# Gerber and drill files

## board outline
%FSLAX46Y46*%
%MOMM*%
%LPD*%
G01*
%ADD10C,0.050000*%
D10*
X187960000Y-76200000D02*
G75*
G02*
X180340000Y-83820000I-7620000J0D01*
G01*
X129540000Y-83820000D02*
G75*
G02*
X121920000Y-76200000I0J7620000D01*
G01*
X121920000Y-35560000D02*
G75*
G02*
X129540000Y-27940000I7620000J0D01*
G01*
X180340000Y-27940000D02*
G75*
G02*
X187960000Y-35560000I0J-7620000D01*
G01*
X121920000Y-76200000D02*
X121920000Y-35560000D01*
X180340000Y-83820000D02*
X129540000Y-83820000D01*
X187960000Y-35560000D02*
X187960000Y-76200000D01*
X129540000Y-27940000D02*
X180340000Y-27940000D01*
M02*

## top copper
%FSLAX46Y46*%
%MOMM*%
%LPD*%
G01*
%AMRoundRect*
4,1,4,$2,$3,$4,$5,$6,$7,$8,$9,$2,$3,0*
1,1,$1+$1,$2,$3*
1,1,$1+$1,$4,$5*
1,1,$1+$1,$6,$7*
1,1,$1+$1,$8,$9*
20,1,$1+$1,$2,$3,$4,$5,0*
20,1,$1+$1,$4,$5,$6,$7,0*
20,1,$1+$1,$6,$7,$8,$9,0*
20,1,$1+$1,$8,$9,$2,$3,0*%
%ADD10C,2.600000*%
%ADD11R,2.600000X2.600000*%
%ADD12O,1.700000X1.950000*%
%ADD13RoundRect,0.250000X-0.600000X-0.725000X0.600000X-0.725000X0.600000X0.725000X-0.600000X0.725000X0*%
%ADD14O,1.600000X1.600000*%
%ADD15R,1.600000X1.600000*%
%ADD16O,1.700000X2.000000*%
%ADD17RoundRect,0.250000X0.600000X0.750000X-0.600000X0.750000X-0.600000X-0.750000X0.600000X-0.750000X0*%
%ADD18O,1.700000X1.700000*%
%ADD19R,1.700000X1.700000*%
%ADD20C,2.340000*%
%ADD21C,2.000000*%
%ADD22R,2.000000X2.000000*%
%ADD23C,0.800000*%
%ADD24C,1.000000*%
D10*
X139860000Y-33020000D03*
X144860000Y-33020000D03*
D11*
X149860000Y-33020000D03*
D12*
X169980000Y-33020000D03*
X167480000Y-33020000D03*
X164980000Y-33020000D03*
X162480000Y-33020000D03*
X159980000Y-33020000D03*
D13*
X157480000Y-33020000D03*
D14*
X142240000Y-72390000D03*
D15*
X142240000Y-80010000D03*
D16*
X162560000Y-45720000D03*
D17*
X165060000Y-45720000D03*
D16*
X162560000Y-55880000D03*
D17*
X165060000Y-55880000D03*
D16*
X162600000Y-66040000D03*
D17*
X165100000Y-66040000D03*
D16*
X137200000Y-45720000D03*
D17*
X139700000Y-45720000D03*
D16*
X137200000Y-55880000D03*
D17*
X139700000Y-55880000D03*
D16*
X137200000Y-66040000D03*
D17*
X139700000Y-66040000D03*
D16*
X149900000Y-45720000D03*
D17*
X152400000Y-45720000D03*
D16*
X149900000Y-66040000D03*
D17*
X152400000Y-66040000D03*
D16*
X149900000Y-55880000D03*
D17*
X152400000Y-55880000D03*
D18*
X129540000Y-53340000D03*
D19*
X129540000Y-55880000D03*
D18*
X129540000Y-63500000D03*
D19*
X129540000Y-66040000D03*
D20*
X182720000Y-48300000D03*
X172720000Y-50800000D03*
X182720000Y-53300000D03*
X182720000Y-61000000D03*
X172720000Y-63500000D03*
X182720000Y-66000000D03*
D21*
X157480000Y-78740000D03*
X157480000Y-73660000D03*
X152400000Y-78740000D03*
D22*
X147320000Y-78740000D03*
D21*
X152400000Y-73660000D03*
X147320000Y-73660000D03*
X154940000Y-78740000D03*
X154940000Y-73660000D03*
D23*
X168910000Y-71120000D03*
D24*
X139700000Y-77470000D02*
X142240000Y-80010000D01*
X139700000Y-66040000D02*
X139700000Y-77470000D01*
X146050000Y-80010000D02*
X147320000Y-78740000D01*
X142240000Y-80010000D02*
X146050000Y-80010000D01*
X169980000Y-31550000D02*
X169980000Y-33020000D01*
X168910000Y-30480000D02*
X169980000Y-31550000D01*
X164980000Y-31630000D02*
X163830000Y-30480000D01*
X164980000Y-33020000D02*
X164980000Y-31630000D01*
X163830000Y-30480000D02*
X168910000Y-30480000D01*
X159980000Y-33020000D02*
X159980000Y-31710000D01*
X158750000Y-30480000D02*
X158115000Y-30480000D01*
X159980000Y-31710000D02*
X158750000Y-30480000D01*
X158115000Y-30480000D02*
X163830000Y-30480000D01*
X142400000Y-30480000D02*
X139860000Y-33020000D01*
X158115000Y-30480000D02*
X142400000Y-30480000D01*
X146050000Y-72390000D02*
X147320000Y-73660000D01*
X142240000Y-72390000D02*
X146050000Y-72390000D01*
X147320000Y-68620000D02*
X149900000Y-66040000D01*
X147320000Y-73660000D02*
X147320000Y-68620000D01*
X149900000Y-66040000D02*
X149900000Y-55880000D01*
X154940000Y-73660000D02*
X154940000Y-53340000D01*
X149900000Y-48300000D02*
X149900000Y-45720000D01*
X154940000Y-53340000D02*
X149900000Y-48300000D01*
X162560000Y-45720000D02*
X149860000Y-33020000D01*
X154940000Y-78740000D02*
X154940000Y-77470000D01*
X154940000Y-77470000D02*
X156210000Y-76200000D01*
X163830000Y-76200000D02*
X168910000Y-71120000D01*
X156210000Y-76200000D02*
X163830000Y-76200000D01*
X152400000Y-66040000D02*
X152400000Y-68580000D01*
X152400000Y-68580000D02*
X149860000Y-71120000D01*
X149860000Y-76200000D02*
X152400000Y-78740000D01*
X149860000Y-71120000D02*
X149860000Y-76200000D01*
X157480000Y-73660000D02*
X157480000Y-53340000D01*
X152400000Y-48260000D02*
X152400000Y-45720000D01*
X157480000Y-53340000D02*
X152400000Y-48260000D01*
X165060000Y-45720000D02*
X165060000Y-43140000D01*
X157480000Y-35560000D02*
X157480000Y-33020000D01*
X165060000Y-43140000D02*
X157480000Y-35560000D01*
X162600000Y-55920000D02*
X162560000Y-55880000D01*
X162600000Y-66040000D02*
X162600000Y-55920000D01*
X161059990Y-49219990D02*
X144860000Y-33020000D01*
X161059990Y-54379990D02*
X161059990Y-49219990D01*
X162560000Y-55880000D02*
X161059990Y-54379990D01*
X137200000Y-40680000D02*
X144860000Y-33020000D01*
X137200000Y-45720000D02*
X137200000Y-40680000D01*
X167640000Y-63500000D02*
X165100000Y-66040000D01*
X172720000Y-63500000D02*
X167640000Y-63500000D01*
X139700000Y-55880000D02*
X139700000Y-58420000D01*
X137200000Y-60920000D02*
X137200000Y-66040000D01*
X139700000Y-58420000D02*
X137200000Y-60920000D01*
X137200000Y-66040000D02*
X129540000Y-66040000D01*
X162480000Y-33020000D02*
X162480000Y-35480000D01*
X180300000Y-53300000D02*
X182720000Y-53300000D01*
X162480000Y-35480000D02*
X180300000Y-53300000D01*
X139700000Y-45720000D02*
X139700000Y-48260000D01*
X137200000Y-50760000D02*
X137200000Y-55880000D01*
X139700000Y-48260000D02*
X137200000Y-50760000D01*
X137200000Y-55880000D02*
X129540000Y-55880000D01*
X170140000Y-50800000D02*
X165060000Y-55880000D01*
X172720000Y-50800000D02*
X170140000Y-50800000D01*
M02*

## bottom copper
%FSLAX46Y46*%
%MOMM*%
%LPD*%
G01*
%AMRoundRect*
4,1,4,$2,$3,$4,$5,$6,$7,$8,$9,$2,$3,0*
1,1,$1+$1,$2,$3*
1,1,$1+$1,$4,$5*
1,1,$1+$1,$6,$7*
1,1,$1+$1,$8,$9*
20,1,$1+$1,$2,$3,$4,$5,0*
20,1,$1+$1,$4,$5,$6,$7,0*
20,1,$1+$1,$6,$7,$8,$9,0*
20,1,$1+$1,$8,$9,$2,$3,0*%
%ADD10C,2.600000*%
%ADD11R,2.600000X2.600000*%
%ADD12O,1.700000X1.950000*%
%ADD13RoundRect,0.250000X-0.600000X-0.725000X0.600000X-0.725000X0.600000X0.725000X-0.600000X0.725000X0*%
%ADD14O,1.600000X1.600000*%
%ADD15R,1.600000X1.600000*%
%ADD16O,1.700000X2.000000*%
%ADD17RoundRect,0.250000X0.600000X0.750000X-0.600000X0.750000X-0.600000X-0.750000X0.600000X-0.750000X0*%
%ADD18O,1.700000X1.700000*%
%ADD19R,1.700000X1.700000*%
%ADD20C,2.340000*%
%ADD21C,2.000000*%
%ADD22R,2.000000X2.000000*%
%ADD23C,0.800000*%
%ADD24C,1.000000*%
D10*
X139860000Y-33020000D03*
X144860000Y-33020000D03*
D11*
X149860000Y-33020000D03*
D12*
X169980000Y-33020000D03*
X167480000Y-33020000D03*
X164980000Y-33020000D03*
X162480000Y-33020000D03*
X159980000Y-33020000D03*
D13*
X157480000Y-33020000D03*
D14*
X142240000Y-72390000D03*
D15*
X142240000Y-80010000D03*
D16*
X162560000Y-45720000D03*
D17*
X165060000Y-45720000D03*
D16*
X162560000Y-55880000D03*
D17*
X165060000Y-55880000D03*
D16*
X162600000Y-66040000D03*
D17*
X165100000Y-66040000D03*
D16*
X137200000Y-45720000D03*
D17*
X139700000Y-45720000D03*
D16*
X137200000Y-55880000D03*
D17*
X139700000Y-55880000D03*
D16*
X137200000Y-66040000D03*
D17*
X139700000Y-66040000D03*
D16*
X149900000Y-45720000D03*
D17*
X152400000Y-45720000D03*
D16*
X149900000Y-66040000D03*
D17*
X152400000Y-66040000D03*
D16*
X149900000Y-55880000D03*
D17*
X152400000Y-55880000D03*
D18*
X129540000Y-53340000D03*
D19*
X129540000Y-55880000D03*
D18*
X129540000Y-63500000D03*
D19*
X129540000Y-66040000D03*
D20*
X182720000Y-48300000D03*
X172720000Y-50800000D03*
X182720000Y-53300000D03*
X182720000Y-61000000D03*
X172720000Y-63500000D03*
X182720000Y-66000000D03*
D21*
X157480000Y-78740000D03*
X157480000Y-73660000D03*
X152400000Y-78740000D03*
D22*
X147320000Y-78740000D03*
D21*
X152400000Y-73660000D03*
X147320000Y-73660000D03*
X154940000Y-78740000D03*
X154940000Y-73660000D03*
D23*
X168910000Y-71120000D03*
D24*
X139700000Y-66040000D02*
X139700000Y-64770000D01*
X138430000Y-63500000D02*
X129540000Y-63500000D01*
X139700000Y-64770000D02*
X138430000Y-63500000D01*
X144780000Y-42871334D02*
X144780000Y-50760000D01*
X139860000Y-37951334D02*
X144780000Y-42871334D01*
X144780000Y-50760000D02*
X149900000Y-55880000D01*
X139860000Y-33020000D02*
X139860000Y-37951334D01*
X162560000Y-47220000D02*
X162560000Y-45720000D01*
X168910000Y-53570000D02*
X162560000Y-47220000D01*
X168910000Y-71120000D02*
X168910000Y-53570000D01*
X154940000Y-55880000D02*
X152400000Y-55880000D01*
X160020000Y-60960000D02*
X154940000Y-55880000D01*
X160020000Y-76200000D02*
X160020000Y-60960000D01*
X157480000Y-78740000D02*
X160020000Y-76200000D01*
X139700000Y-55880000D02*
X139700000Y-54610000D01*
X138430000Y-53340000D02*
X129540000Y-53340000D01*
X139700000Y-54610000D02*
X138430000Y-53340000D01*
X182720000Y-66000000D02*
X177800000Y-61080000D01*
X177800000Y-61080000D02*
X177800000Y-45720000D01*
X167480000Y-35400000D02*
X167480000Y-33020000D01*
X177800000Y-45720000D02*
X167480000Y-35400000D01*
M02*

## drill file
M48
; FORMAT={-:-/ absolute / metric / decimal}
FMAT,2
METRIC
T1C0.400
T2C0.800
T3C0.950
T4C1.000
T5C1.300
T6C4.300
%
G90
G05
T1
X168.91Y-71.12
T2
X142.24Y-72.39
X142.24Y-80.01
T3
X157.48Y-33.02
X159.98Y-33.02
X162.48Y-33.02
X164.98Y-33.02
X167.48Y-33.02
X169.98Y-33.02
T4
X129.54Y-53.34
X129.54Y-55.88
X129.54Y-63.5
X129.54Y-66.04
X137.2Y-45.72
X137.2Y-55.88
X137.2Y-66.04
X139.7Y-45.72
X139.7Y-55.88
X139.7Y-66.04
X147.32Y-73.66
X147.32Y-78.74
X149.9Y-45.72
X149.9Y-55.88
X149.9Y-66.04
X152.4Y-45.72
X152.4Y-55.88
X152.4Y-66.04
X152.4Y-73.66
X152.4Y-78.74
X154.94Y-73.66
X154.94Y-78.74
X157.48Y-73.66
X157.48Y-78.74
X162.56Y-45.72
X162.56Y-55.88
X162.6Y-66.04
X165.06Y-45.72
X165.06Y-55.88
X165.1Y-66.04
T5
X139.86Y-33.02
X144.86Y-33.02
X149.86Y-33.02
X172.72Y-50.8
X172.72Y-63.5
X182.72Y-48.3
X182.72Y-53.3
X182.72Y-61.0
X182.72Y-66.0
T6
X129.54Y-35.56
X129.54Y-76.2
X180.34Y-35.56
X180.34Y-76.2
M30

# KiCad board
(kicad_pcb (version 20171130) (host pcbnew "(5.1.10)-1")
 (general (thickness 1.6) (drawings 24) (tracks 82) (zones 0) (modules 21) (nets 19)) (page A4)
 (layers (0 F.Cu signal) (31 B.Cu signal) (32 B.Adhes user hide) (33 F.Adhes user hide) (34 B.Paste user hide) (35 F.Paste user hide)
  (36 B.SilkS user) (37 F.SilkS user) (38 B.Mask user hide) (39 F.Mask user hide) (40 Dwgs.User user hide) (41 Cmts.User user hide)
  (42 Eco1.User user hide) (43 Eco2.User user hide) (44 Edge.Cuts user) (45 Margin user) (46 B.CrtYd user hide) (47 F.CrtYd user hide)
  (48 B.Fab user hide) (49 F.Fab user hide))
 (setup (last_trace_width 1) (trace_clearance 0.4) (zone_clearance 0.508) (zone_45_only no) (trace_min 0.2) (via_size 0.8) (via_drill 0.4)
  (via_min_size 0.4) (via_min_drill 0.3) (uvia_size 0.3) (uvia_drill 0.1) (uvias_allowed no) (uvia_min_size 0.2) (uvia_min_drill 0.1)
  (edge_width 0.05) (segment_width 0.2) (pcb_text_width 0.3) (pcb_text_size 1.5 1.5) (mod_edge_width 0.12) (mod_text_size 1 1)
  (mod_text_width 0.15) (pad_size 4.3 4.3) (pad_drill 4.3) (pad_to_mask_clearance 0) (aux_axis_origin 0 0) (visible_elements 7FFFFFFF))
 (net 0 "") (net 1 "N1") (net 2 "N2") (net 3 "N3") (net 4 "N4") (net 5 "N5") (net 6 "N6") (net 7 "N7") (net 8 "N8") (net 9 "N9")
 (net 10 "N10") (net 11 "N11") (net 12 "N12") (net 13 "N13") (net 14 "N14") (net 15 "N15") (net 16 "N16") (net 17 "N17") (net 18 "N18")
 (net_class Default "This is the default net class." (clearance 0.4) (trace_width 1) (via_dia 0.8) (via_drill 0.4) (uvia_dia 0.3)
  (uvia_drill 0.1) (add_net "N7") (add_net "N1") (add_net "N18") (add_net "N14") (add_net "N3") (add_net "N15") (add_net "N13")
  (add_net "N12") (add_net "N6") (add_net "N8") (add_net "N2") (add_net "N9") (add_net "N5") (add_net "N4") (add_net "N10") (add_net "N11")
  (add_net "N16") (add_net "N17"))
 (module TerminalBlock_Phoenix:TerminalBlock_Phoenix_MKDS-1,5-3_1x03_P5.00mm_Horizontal (layer F.Cu) (at 149.86 33.02 180)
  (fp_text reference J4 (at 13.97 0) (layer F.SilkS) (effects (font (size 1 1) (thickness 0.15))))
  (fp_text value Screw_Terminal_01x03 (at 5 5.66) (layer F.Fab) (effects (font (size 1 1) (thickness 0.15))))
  (pad 3 thru_hole circle (at 10 0 180) (size 2.6 2.6) (drill 1.3) (layers *.Cu *.Mask) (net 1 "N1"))
  (pad 2 thru_hole circle (at 5 0 180) (size 2.6 2.6) (drill 1.3) (layers *.Cu *.Mask) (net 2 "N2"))
  (pad 1 thru_hole rect (at 0 0 180) (size 2.6 2.6) (drill 1.3) (layers *.Cu *.Mask) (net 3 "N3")))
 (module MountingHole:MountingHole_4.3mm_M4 (layer F.Cu) (at 180.34 76.2)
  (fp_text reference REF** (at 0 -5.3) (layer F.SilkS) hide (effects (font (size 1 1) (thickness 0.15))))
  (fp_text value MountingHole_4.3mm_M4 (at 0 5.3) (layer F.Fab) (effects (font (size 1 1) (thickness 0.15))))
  (pad 1 np_thru_hole circle (at 0 0) (size 4.3 4.3) (drill 4.3) (layers *.Cu *.Mask)))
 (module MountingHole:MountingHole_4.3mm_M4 (layer F.Cu) (at 129.54 76.2)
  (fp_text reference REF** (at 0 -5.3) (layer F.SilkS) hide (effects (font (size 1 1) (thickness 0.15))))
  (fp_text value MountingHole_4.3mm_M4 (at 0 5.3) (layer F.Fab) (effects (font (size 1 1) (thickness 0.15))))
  (pad 1 np_thru_hole circle (at 0 0) (size 4.3 4.3) (drill 4.3) (layers *.Cu *.Mask)))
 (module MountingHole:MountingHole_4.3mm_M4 (layer F.Cu) (at 129.54 35.56)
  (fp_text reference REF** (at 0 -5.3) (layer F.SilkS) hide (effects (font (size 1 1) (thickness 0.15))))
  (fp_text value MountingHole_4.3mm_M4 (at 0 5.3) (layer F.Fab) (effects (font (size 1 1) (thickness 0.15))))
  (pad 1 np_thru_hole circle (at 0 0) (size 4.3 4.3) (drill 4.3) (layers *.Cu *.Mask)))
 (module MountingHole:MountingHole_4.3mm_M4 (layer F.Cu) (at 180.34 35.56)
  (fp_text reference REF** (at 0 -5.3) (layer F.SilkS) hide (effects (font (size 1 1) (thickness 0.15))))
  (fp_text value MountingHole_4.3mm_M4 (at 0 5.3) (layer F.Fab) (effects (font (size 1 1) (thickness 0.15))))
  (pad 1 np_thru_hole circle (at 0 0) (size 4.3 4.3) (drill 4.3) (layers *.Cu *.Mask)))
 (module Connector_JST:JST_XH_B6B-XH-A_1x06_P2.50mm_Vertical (layer F.Cu) (at 157.48 33.02)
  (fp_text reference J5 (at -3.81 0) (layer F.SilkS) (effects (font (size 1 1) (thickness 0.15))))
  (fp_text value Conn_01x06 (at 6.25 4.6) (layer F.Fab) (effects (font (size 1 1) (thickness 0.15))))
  (pad 6 thru_hole oval (at 12.5 0) (size 1.7 1.95) (drill 0.95) (layers *.Cu *.Mask) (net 1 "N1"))
  (pad 5 thru_hole oval (at 10 0) (size 1.7 1.95) (drill 0.95) (layers *.Cu *.Mask) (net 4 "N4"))
  (pad 4 thru_hole oval (at 7.5 0) (size 1.7 1.95) (drill 0.95) (layers *.Cu *.Mask) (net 1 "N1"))
  (pad 3 thru_hole oval (at 5 0) (size 1.7 1.95) (drill 0.95) (layers *.Cu *.Mask) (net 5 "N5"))
  (pad 2 thru_hole oval (at 2.5 0) (size 1.7 1.95) (drill 0.95) (layers *.Cu *.Mask) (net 1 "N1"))
  (pad 1 thru_hole roundrect (at 0 0) (size 1.7 1.95) (drill 0.95) (layers *.Cu *.Mask) (roundrect_rratio 0.147059) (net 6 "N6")))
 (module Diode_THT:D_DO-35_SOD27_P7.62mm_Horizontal (layer F.Cu) (at 142.24 80.01 90)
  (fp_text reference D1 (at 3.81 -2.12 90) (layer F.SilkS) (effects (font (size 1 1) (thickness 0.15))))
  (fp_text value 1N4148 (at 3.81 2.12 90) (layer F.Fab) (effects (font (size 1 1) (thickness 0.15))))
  (pad 2 thru_hole oval (at 7.62 0 90) (size 1.6 1.6) (drill 0.8) (layers *.Cu *.Mask) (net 1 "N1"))
  (pad 1 thru_hole rect (at 0 0 90) (size 1.6 1.6) (drill 0.8) (layers *.Cu *.Mask) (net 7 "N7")))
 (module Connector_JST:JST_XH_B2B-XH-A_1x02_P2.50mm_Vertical (layer F.Cu) (at 165.06 45.72 180)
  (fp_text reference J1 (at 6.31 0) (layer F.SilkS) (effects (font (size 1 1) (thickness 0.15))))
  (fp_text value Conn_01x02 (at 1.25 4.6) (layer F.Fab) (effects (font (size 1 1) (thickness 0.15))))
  (pad 2 thru_hole oval (at 2.5 0 180) (size 1.7 2) (drill 1) (layers *.Cu *.Mask) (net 3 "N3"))
  (pad 1 thru_hole roundrect (at 0 0 180) (size 1.7 2) (drill 1) (layers *.Cu *.Mask) (roundrect_rratio 0.147059) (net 6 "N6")))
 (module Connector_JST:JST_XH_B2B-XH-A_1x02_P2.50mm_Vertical (layer F.Cu) (at 165.06 55.88 180)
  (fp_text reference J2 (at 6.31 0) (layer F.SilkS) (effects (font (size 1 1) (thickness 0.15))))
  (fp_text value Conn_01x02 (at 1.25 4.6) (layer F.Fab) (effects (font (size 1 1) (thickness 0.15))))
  (pad 2 thru_hole oval (at 2.5 0 180) (size 1.7 2) (drill 1) (layers *.Cu *.Mask) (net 2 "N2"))
  (pad 1 thru_hole roundrect (at 0 0 180) (size 1.7 2) (drill 1) (layers *.Cu *.Mask) (roundrect_rratio 0.147059) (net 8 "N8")))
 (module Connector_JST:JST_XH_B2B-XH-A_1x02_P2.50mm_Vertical (layer F.Cu) (at 165.1 66.04 180)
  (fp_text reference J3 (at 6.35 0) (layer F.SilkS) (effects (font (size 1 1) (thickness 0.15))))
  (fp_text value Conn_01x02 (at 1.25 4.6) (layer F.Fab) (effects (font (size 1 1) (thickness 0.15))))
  (pad 2 thru_hole oval (at 2.5 0 180) (size 1.7 2) (drill 1) (layers *.Cu *.Mask) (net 2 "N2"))
  (pad 1 thru_hole roundrect (at 0 0 180) (size 1.7 2) (drill 1) (layers *.Cu *.Mask) (roundrect_rratio 0.147059) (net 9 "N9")))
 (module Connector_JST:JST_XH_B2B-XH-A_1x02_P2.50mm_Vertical (layer F.Cu) (at 139.7 45.72 180)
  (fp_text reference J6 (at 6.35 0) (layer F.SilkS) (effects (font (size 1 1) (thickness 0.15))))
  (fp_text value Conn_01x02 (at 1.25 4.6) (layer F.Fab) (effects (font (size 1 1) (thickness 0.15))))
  (pad 2 thru_hole oval (at 2.5 0 180) (size 1.7 2) (drill 1) (layers *.Cu *.Mask) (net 2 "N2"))
  (pad 1 thru_hole roundrect (at 0 0 180) (size 1.7 2) (drill 1) (layers *.Cu *.Mask) (roundrect_rratio 0.147059) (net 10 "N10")))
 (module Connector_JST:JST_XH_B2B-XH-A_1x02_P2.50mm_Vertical (layer F.Cu) (at 139.7 55.88 180)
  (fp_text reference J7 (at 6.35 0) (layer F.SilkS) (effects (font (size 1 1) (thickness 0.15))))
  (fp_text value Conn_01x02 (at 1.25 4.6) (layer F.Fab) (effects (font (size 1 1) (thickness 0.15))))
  (pad 2 thru_hole oval (at 2.5 0 180) (size 1.7 2) (drill 1) (layers *.Cu *.Mask) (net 10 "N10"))
  (pad 1 thru_hole roundrect (at 0 0 180) (size 1.7 2) (drill 1) (layers *.Cu *.Mask) (roundrect_rratio 0.147059) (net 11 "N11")))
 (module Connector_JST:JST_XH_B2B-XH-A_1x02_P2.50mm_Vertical (layer F.Cu) (at 139.7 66.04 180)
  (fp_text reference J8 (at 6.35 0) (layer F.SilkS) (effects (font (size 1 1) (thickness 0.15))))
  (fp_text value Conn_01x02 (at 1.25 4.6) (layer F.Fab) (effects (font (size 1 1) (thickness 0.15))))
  (pad 2 thru_hole oval (at 2.5 0 180) (size 1.7 2) (drill 1) (layers *.Cu *.Mask) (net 11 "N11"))
  (pad 1 thru_hole roundrect (at 0 0 180) (size 1.7 2) (drill 1) (layers *.Cu *.Mask) (roundrect_rratio 0.147059) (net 7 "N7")))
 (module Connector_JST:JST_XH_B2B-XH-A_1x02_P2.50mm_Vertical (layer F.Cu) (at 152.4 45.72 180)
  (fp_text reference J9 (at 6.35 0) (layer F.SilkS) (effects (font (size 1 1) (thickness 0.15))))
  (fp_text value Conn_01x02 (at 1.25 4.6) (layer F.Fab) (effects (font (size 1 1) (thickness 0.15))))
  (pad 2 thru_hole oval (at 2.5 0 180) (size 1.7 2) (drill 1) (layers *.Cu *.Mask) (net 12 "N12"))
  (pad 1 thru_hole roundrect (at 0 0 180) (size 1.7 2) (drill 1) (layers *.Cu *.Mask) (roundrect_rratio 0.147059) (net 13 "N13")))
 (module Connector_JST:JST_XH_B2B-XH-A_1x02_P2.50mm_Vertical (layer F.Cu) (at 152.4 66.04 180)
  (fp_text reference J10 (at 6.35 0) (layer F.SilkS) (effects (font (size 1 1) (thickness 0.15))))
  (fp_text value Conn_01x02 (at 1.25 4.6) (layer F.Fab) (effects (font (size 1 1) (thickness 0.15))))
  (pad 2 thru_hole oval (at 2.5 0 180) (size 1.7 2) (drill 1) (layers *.Cu *.Mask) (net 1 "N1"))
  (pad 1 thru_hole roundrect (at 0 0 180) (size 1.7 2) (drill 1) (layers *.Cu *.Mask) (roundrect_rratio 0.147059) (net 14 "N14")))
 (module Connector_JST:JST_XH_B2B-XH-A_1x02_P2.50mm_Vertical (layer F.Cu) (at 152.4 55.88 180)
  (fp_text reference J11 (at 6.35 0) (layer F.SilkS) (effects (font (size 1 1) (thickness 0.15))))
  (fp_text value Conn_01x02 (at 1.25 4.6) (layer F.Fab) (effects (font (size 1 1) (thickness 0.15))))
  (pad 2 thru_hole oval (at 2.5 0 180) (size 1.7 2) (drill 1) (layers *.Cu *.Mask) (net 1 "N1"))
  (pad 1 thru_hole roundrect (at 0 0 180) (size 1.7 2) (drill 1) (layers *.Cu *.Mask) (roundrect_rratio 0.147059) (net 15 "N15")))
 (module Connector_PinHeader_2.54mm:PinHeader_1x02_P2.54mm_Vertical (layer F.Cu) (at 129.54 55.88 180)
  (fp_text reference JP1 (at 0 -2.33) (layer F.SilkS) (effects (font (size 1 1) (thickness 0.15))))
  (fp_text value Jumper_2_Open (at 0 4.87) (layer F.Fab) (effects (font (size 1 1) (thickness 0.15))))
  (pad 2 thru_hole oval (at 0 2.54 180) (size 1.7 1.7) (drill 1) (layers *.Cu *.Mask) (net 11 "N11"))
  (pad 1 thru_hole rect (at 0 0 180) (size 1.7 1.7) (drill 1) (layers *.Cu *.Mask) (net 10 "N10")))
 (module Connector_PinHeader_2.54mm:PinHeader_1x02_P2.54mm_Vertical (layer F.Cu) (at 129.54 66.04 180)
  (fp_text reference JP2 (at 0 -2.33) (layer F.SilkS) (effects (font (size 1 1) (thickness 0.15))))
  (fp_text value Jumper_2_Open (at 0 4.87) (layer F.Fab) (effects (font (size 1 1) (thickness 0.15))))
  (pad 2 thru_hole oval (at 0 2.54 180) (size 1.7 1.7) (drill 1) (layers *.Cu *.Mask) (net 7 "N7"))
  (pad 1 thru_hole rect (at 0 0 180) (size 1.7 1.7) (drill 1) (layers *.Cu *.Mask) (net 11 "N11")))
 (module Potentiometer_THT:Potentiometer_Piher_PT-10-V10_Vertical (layer F.Cu) (at 182.72 48.3 180)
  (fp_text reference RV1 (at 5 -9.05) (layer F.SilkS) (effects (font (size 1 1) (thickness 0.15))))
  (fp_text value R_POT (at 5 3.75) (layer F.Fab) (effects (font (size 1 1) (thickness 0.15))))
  (pad 1 thru_hole circle (at 0 0 180) (size 2.34 2.34) (drill 1.3) (layers *.Cu *.Mask) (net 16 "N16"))
  (pad 2 thru_hole circle (at 10 -2.5 180) (size 2.34 2.34) (drill 1.3) (layers *.Cu *.Mask) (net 8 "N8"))
  (pad 3 thru_hole circle (at 0 -5 180) (size 2.34 2.34) (drill 1.3) (layers *.Cu *.Mask) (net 5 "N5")))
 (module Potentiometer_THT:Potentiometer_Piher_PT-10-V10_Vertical (layer F.Cu) (at 182.72 61 180)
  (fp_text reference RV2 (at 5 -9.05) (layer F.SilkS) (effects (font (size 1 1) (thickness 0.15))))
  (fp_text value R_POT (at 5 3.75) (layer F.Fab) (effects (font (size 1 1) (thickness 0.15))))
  (pad 1 thru_hole circle (at 0 0 180) (size 2.34 2.34) (drill 1.3) (layers *.Cu *.Mask) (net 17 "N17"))
  (pad 2 thru_hole circle (at 10 -2.5 180) (size 2.34 2.34) (drill 1.3) (layers *.Cu *.Mask) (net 9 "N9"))
  (pad 3 thru_hole circle (at 0 -5 180) (size 2.34 2.34) (drill 1.3) (layers *.Cu *.Mask) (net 4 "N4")))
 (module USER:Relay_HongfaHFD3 (layer F.Cu) (at 147.32 78.74 90)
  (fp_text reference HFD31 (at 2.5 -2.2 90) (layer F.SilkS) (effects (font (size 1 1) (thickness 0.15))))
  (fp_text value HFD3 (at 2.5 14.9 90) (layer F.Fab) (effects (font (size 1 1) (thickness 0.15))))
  (pad 5 thru_hole circle (at 0 10.16 90) (size 2 2) (drill 1) (layers *.Cu *.Mask) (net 15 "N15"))
  (pad 8 thru_hole circle (at 5.08 10.16 90) (size 2 2) (drill 1) (layers *.Cu *.Mask) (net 13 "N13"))
  (pad 3 thru_hole circle (at 0 5.08 90) (size 2 2) (drill 1) (layers *.Cu *.Mask) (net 14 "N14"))
  (pad 1 thru_hole rect (at 0 0 90) (size 2 2) (drill 1) (layers *.Cu *.Mask) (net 7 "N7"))
  (pad 10 thru_hole circle (at 5.08 5.08 90) (size 2 2) (drill 1) (layers *.Cu *.Mask) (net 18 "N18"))
  (pad 12 thru_hole circle (at 5.08 0 90) (size 2 2) (drill 1) (layers *.Cu *.Mask) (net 1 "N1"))
  (pad 4 thru_hole circle (at 0 7.62) (size 2 2) (drill 1) (layers *.Cu *.Mask) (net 3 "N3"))
  (pad 9 thru_hole circle (at 5.08 7.62) (size 2 2) (drill 1) (layers *.Cu *.Mask) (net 12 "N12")))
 (gr_arc (start 180.34 76.2) (end 180.34 83.82) (angle -90) (layer Edge.Cuts) (width 0.05))
 (gr_arc (start 129.54 76.2) (end 121.92 76.2) (angle -90) (layer Edge.Cuts) (width 0.05))
 (gr_arc (start 129.54 35.56) (end 129.54 27.94) (angle -90) (layer Edge.Cuts) (width 0.05))
 (gr_arc (start 180.34 35.56) (end 187.96 35.56) (angle -90) (layer Edge.Cuts) (width 0.05))
 (gr_line (start 121.92 76.2) (end 121.92 35.56) (layer Edge.Cuts) (width 0.05))
 (gr_line (start 180.34 83.82) (end 129.54 83.82) (layer Edge.Cuts) (width 0.05))
 (gr_line (start 187.96 35.56) (end 187.96 76.2) (layer Edge.Cuts) (width 0.05))
 (gr_line (start 129.54 27.94) (end 180.34 27.94) (layer Edge.Cuts) (width 0.05))
 (segment (start 139.7 77.47) (end 142.24 80.01) (width 1) (layer F.Cu) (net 7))
 (segment (start 139.7 66.04) (end 139.7 77.47) (width 1) (layer F.Cu) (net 7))
 (segment (start 146.05 80.01) (end 147.32 78.74) (width 1) (layer F.Cu) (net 7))
 (segment (start 142.24 80.01) (end 146.05 80.01) (width 1) (layer F.Cu) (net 7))
 (segment (start 139.7 66.04) (end 139.7 64.77) (width 1) (layer B.Cu) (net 7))
 (segment (start 138.43 63.5) (end 129.54 63.5) (width 1) (layer B.Cu) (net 7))
 (segment (start 139.7 64.77) (end 138.43 63.5) (width 1) (layer B.Cu) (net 7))
 (segment (start 169.98 31.55) (end 169.98 33.02) (width 1) (layer F.Cu) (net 1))
 (segment (start 168.91 30.48) (end 169.98 31.55) (width 1) (layer F.Cu) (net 1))
 (segment (start 164.98 31.63) (end 163.83 30.48) (width 1) (layer F.Cu) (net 1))
 (segment (start 164.98 33.02) (end 164.98 31.63) (width 1) (layer F.Cu) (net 1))
 (segment (start 163.83 30.48) (end 168.91 30.48) (width 1) (layer F.Cu) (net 1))
 (segment (start 159.98 33.02) (end 159.98 31.71) (width 1) (layer F.Cu) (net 1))
 (segment (start 158.75 30.48) (end 158.115 30.48) (width 1) (layer F.Cu) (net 1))
 (segment (start 159.98 31.71) (end 158.75 30.48) (width 1) (layer F.Cu) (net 1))
 (segment (start 158.115 30.48) (end 163.83 30.48) (width 1) (layer F.Cu) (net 1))
 (segment (start 142.4 30.48) (end 139.86 33.02) (width 1) (layer F.Cu) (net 1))
 (segment (start 158.115 30.48) (end 142.4 30.48) (width 1) (layer F.Cu) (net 1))
 (segment (start 146.05 72.39) (end 147.32 73.66) (width 1) (layer F.Cu) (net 1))
 (segment (start 142.24 72.39) (end 146.05 72.39) (width 1) (layer F.Cu) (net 1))
 (segment (start 147.32 68.62) (end 149.9 66.04) (width 1) (layer F.Cu) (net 1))
 (segment (start 147.32 73.66) (end 147.32 68.62) (width 1) (layer F.Cu) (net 1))
 (segment (start 149.9 66.04) (end 149.9 55.88) (width 1) (layer F.Cu) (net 1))
 (segment (start 144.78 42.871334) (end 144.78 50.76) (width 1) (layer B.Cu) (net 1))
 (segment (start 139.86 37.951334) (end 144.78 42.871334) (width 1) (layer B.Cu) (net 1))
 (segment (start 144.78 50.76) (end 149.9 55.88) (width 1) (layer B.Cu) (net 1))
 (segment (start 139.86 33.02) (end 139.86 37.951334) (width 1) (layer B.Cu) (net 1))
 (segment (start 154.94 73.66) (end 154.94 53.34) (width 1) (layer F.Cu) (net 12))
 (segment (start 149.9 48.3) (end 149.9 45.72) (width 1) (layer F.Cu) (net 12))
 (segment (start 154.94 53.34) (end 149.9 48.3) (width 1) (layer F.Cu) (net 12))
 (segment (start 162.56 45.72) (end 149.86 33.02) (width 1) (layer F.Cu) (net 3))
 (segment (start 154.94 78.74) (end 154.94 77.47) (width 1) (layer F.Cu) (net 3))
 (segment (start 154.94 77.47) (end 156.21 76.2) (width 1) (layer F.Cu) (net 3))
 (via (at 168.91 71.12) (size 0.8) (drill 0.4) (layers F.Cu B.Cu) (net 3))
 (segment (start 163.83 76.2) (end 168.91 71.12) (width 1) (layer F.Cu) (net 3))
 (segment (start 156.21 76.2) (end 163.83 76.2) (width 1) (layer F.Cu) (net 3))
 (segment (start 162.56 47.22) (end 162.56 45.72) (width 1) (layer B.Cu) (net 3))
 (segment (start 168.91 53.57) (end 162.56 47.22) (width 1) (layer B.Cu) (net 3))
 (segment (start 168.91 71.12) (end 168.91 53.57) (width 1) (layer B.Cu) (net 3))
 (segment (start 152.4 66.04) (end 152.4 68.58) (width 1) (layer F.Cu) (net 14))
 (segment (start 152.4 68.58) (end 149.86 71.12) (width 1) (layer F.Cu) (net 14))
 (segment (start 149.86 76.2) (end 152.4 78.74) (width 1) (layer F.Cu) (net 14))
 (segment (start 149.86 71.12) (end 149.86 76.2) (width 1) (layer F.Cu) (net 14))
 (segment (start 157.48 73.66) (end 157.48 53.34) (width 1) (layer F.Cu) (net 13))
 (segment (start 152.4 48.26) (end 152.4 45.72) (width 1) (layer F.Cu) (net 13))
 (segment (start 157.48 53.34) (end 152.4 48.26) (width 1) (layer F.Cu) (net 13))
 (segment (start 154.94 55.88) (end 152.4 55.88) (width 1) (layer B.Cu) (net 15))
 (segment (start 160.02 60.96) (end 154.94 55.88) (width 1) (layer B.Cu) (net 15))
 (segment (start 160.02 76.2) (end 160.02 60.96) (width 1) (layer B.Cu) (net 15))
 (segment (start 157.48 78.74) (end 160.02 76.2) (width 1) (layer B.Cu) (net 15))
 (segment (start 165.06 45.72) (end 165.06 43.14) (width 1) (layer F.Cu) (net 6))
 (segment (start 157.48 35.56) (end 157.48 33.02) (width 1) (layer F.Cu) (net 6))
 (segment (start 165.06 43.14) (end 157.48 35.56) (width 1) (layer F.Cu) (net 6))
 (segment (start 162.6 55.92) (end 162.56 55.88) (width 1) (layer F.Cu) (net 2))
 (segment (start 162.6 66.04) (end 162.6 55.92) (width 1) (layer F.Cu) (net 2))
 (segment (start 161.05999 49.21999) (end 144.86 33.02) (width 1) (layer F.Cu) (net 2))
 (segment (start 161.05999 54.37999) (end 161.05999 49.21999) (width 1) (layer F.Cu) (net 2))
 (segment (start 162.56 55.88) (end 161.05999 54.37999) (width 1) (layer F.Cu) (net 2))
 (segment (start 137.2 40.68) (end 144.86 33.02) (width 1) (layer F.Cu) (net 2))
 (segment (start 137.2 45.72) (end 137.2 40.68) (width 1) (layer F.Cu) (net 2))
 (segment (start 167.64 63.5) (end 165.1 66.04) (width 1) (layer F.Cu) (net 9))
 (segment (start 172.72 63.5) (end 167.64 63.5) (width 1) (layer F.Cu) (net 9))
 (segment (start 139.7 55.88) (end 139.7 58.42) (width 1) (layer F.Cu) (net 11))
 (segment (start 137.2 60.92) (end 137.2 66.04) (width 1) (layer F.Cu) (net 11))
 (segment (start 139.7 58.42) (end 137.2 60.92) (width 1) (layer F.Cu) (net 11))
 (segment (start 137.2 66.04) (end 129.54 66.04) (width 1) (layer F.Cu) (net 11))
 (segment (start 139.7 55.88) (end 139.7 54.61) (width 1) (layer B.Cu) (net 11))
 (segment (start 138.43 53.34) (end 129.54 53.34) (width 1) (layer B.Cu) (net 11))
 (segment (start 139.7 54.61) (end 138.43 53.34) (width 1) (layer B.Cu) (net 11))
 (segment (start 162.48 33.02) (end 162.48 35.48) (width 1) (layer F.Cu) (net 5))
 (segment (start 180.3 53.3) (end 182.72 53.3) (width 1) (layer F.Cu) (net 5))
 (segment (start 162.48 35.48) (end 180.3 53.3) (width 1) (layer F.Cu) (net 5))
 (segment (start 182.72 66) (end 177.8 61.08) (width 1) (layer B.Cu) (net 4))
 (segment (start 177.8 61.08) (end 177.8 45.72) (width 1) (layer B.Cu) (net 4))
 (segment (start 167.48 35.4) (end 167.48 33.02) (width 1) (layer B.Cu) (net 4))
 (segment (start 177.8 45.72) (end 167.48 35.4) (width 1) (layer B.Cu) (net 4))
 (segment (start 139.7 45.72) (end 139.7 48.26) (width 1) (layer F.Cu) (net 10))
 (segment (start 137.2 50.76) (end 137.2 55.88) (width 1) (layer F.Cu) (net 10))
 (segment (start 139.7 48.26) (end 137.2 50.76) (width 1) (layer F.Cu) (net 10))
 (segment (start 137.2 55.88) (end 129.54 55.88) (width 1) (layer F.Cu) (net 10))
 (segment (start 170.14 50.8) (end 165.06 55.88) (width 1) (layer F.Cu) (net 8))
 (segment (start 172.72 50.8) (end 170.14 50.8) (width 1) (layer F.Cu) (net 8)))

